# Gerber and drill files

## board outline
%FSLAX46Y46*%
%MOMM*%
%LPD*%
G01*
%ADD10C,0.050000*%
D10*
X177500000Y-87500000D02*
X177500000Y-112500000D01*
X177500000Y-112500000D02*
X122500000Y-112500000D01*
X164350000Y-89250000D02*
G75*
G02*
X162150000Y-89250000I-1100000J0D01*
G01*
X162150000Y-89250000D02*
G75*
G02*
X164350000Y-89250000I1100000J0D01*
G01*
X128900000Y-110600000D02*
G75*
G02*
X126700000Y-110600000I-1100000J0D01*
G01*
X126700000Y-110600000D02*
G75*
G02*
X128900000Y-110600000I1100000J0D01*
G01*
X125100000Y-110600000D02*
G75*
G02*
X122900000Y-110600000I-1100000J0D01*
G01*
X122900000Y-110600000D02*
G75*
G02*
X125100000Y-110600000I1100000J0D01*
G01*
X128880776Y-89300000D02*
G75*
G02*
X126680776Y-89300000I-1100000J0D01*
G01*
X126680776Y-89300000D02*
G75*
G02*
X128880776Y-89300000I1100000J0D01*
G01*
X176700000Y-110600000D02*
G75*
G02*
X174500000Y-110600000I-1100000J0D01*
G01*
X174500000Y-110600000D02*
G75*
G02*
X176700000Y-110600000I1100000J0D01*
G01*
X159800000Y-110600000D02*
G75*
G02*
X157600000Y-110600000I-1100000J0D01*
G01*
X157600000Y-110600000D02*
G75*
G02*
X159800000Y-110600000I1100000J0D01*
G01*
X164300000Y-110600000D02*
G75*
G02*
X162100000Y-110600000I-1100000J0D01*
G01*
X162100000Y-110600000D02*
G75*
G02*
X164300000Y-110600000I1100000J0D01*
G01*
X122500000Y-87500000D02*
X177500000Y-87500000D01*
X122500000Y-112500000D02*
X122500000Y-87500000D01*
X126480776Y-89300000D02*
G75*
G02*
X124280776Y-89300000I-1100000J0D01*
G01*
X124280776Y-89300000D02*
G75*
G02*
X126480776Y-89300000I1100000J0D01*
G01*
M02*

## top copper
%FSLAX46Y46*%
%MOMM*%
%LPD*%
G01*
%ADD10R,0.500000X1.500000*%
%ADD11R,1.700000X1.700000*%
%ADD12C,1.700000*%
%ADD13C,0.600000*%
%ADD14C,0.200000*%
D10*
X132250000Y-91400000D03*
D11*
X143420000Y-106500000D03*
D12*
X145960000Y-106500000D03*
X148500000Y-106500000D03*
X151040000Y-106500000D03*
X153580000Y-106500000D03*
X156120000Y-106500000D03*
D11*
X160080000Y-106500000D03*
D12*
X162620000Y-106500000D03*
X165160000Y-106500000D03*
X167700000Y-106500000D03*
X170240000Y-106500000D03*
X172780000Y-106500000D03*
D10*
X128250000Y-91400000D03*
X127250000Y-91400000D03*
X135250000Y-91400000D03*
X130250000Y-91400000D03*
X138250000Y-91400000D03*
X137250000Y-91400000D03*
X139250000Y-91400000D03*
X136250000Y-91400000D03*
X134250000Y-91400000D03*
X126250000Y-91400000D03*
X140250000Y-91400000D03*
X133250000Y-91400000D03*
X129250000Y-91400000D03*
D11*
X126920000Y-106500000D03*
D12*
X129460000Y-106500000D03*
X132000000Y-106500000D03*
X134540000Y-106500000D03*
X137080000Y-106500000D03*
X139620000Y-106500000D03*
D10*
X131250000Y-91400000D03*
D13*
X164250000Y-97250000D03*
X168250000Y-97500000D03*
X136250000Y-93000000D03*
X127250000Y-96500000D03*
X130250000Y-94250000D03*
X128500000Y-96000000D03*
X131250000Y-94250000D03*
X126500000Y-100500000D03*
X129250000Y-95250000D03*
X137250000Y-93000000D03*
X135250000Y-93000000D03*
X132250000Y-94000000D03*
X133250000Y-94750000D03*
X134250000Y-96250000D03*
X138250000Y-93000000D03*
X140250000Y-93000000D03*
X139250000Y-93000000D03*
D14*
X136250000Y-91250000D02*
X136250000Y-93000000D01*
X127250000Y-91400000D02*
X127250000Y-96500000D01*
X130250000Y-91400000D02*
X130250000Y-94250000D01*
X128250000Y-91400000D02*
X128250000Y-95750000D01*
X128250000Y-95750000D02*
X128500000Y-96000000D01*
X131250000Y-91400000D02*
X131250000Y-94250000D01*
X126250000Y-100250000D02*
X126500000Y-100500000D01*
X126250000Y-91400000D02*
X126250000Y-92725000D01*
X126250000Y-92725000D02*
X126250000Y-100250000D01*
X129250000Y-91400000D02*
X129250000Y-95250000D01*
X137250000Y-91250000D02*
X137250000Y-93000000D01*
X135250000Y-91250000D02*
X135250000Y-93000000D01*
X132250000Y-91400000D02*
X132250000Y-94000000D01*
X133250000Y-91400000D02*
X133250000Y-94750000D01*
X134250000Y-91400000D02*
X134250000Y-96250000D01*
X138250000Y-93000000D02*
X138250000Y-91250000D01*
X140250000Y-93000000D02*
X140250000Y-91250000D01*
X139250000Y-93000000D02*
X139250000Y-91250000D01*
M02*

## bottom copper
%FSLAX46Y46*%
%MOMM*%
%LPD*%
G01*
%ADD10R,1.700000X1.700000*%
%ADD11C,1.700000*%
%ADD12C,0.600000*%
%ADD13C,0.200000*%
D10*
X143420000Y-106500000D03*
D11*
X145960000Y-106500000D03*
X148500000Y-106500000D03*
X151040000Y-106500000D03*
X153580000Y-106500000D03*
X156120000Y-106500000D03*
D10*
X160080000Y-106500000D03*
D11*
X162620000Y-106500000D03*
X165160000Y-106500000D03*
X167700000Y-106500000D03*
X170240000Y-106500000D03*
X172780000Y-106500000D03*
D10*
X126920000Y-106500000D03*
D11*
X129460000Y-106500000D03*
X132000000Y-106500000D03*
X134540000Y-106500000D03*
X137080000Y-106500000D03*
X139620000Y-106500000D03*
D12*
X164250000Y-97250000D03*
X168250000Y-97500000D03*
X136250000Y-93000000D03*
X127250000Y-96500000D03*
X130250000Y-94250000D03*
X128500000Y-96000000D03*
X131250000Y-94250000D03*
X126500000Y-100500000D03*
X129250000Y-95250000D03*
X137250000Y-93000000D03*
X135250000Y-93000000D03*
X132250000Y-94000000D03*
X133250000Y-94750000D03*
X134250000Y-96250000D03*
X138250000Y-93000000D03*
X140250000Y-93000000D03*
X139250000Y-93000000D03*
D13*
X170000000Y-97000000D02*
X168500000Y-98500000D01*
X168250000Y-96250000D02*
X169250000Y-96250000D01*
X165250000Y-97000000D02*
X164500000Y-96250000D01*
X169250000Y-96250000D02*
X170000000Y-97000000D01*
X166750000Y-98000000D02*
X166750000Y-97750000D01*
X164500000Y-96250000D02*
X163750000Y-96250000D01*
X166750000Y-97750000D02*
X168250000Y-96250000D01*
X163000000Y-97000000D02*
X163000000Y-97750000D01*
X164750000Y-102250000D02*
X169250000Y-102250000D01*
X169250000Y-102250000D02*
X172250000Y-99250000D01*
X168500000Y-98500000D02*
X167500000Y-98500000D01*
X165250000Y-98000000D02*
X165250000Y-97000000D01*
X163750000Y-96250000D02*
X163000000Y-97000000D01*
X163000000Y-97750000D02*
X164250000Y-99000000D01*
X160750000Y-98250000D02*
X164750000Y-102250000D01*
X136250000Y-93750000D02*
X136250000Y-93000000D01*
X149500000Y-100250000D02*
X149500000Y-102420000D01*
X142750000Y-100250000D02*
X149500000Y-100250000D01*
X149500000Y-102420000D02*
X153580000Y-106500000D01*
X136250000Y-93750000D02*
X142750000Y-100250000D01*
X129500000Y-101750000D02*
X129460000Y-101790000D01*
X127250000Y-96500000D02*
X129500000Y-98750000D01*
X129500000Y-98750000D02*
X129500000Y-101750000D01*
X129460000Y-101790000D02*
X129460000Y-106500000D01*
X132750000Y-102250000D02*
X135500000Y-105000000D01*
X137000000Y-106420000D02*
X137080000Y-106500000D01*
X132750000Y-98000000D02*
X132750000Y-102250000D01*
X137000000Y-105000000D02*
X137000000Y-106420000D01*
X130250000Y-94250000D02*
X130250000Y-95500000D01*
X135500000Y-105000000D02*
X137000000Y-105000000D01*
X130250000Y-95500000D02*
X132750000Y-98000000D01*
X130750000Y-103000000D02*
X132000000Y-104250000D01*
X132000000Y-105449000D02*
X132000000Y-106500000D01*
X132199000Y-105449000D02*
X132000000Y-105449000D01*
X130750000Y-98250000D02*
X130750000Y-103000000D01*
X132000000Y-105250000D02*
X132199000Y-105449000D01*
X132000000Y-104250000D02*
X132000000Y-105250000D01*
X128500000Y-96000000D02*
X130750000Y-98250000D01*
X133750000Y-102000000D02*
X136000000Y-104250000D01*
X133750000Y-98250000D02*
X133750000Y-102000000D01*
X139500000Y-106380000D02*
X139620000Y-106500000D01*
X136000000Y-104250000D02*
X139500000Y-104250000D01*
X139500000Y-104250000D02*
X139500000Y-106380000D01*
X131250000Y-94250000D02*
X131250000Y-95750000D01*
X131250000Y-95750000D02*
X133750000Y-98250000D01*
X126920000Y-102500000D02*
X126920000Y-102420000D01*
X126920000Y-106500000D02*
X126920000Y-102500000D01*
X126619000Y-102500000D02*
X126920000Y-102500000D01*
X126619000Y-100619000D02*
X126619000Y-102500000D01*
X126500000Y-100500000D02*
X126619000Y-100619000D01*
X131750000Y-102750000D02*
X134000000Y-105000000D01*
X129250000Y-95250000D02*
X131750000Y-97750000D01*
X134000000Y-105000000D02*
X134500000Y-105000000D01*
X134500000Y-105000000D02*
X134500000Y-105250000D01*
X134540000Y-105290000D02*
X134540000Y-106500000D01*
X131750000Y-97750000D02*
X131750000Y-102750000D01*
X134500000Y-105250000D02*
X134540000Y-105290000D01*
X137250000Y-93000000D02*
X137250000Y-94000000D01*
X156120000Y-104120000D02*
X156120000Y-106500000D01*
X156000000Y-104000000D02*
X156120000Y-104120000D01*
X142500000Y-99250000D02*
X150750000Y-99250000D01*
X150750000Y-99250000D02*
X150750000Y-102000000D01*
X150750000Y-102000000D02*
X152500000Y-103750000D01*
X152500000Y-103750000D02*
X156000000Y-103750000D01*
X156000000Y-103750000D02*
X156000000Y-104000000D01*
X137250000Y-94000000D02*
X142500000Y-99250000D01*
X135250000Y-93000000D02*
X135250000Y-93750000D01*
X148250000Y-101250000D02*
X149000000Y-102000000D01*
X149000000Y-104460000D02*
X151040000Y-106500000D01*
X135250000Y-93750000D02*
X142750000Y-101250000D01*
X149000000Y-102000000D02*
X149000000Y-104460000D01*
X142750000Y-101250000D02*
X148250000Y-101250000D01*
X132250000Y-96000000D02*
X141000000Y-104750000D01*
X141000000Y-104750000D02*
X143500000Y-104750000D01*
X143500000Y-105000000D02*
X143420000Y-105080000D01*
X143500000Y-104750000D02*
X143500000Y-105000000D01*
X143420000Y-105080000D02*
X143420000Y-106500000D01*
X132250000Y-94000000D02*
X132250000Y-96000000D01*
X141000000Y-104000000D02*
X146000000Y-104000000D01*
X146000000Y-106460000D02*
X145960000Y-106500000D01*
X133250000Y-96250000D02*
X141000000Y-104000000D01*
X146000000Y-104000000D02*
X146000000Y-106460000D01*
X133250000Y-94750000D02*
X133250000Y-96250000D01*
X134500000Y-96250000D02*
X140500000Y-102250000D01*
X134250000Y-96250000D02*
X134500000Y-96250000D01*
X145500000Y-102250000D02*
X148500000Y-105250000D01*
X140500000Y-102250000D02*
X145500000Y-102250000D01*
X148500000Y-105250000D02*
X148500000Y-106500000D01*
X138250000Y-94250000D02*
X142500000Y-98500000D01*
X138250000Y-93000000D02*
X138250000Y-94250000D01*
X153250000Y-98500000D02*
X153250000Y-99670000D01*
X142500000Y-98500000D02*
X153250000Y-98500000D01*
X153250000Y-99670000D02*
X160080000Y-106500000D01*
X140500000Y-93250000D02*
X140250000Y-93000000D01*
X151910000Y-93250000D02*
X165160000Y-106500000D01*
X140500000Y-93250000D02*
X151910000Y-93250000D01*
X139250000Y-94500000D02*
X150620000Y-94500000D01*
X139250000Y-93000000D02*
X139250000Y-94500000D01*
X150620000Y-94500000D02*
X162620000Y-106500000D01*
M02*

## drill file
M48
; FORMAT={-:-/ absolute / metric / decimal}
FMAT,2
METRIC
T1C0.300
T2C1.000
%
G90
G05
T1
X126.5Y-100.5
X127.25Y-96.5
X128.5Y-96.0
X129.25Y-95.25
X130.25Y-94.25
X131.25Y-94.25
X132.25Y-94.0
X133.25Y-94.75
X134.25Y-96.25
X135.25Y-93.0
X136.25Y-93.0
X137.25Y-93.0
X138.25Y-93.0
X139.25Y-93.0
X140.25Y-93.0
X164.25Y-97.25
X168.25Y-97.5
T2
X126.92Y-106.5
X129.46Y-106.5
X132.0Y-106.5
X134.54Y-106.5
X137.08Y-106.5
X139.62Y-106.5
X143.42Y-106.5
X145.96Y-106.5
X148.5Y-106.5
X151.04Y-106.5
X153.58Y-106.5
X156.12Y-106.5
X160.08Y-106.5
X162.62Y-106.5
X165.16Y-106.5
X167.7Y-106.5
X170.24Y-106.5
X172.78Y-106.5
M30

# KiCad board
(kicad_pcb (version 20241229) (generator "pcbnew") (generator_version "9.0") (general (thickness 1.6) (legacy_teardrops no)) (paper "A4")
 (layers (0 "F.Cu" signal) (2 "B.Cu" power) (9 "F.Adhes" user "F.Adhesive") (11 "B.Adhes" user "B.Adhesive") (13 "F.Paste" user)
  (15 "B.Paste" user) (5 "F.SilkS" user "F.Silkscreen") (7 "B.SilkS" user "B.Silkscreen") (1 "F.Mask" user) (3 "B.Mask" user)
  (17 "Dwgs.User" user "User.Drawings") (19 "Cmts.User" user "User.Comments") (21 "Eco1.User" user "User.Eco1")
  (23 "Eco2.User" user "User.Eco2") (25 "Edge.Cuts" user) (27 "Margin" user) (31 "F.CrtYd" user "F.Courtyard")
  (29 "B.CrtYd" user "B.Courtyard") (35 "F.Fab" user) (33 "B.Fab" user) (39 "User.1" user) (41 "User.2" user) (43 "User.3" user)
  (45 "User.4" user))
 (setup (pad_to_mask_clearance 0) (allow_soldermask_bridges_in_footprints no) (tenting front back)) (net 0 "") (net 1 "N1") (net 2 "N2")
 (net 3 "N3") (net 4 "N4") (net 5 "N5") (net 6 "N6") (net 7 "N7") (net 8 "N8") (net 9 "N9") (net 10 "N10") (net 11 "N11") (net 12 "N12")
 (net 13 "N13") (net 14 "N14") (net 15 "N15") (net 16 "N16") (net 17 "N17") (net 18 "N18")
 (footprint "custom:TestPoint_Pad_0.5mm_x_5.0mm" (layer "F.Cu") (at 132.25 92.15)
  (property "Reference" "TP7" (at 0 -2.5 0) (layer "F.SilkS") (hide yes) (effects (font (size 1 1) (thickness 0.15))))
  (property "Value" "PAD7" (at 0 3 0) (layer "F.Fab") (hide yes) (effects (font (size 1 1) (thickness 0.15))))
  (pad "1" smd rect (at 0 -0.75) (size 0.5 1.5) (layers "F.Cu" "F.Mask" "F.Paste") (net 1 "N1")))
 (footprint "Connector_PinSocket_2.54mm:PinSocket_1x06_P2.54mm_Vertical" (layer "F.Cu") (at 143.42 106.5 90)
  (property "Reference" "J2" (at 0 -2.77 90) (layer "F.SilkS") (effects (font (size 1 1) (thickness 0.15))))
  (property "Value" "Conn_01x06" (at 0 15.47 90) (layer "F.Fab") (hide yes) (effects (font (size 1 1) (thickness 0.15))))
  (pad "1" thru_hole rect (at 0 0 90) (size 1.7 1.7) (drill 1) (layers "*.Cu" "*.Mask") (remove_unused_layers no) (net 1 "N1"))
  (pad "2" thru_hole circle (at 0 2.54 90) (size 1.7 1.7) (drill 1) (layers "*.Cu" "*.Mask") (remove_unused_layers no) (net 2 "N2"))
  (pad "3" thru_hole circle (at 0 5.08 90) (size 1.7 1.7) (drill 1) (layers "*.Cu" "*.Mask") (remove_unused_layers no) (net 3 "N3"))
  (pad "4" thru_hole circle (at 0 7.62 90) (size 1.7 1.7) (drill 1) (layers "*.Cu" "*.Mask") (remove_unused_layers no) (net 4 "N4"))
  (pad "5" thru_hole circle (at 0 10.16 90) (size 1.7 1.7) (drill 1) (layers "*.Cu" "*.Mask") (remove_unused_layers no) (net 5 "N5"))
  (pad "6" thru_hole circle (at 0 12.7 90) (size 1.7 1.7) (drill 1) (layers "*.Cu" "*.Mask") (remove_unused_layers no) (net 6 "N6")))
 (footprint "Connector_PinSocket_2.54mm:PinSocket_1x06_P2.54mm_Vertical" (layer "F.Cu") (at 160.08 106.5 90)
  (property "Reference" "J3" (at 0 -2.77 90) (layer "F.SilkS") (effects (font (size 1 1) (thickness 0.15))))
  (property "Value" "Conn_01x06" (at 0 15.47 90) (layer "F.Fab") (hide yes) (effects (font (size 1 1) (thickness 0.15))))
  (pad "1" thru_hole rect (at 0 0 90) (size 1.7 1.7) (drill 1) (layers "*.Cu" "*.Mask") (remove_unused_layers no) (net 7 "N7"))
  (pad "2" thru_hole circle (at 0 2.54 90) (size 1.7 1.7) (drill 1) (layers "*.Cu" "*.Mask") (remove_unused_layers no) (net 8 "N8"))
  (pad "3" thru_hole circle (at 0 5.08 90) (size 1.7 1.7) (drill 1) (layers "*.Cu" "*.Mask") (remove_unused_layers no) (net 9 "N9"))
  (pad "4" thru_hole circle (at 0 7.62 90) (size 1.7 1.7) (drill 1) (layers "*.Cu" "*.Mask") (remove_unused_layers no) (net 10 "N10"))
  (pad "5" thru_hole circle (at 0 10.16 90) (size 1.7 1.7) (drill 1) (layers "*.Cu" "*.Mask") (remove_unused_layers no) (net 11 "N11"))
  (pad "6" thru_hole circle (at 0 12.7 90) (size 1.7 1.7) (drill 1) (layers "*.Cu" "*.Mask") (remove_unused_layers no) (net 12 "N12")))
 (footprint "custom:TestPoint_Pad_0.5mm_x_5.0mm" (layer "F.Cu") (at 128.25 92.15)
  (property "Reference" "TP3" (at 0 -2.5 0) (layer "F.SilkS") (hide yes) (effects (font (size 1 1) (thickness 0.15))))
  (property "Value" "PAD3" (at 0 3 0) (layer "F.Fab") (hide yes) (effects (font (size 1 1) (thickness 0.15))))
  (pad "1" smd rect (at 0 -0.75) (size 0.5 1.5) (layers "F.Cu" "F.Mask" "F.Paste") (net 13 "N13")))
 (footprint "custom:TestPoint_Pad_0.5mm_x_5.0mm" (layer "F.Cu") (at 127.25 92.15)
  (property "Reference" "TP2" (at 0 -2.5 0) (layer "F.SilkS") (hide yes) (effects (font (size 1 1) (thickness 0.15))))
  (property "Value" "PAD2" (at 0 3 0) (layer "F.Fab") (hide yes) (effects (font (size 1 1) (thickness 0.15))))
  (pad "1" smd rect (at 0 -0.75) (size 0.5 1.5) (layers "F.Cu" "F.Mask" "F.Paste") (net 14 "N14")))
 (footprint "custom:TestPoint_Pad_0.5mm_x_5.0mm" (layer "F.Cu") (at 135.25 92.15)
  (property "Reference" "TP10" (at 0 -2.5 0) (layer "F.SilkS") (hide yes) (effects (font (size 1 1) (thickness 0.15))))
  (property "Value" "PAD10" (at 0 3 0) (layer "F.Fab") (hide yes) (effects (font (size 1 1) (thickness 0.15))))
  (pad "1" smd rect (at 0 -0.75) (size 0.5 1.5) (layers "F.Cu" "F.Mask" "F.Paste") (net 4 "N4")))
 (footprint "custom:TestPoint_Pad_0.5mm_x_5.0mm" (layer "F.Cu") (at 130.25 92.15)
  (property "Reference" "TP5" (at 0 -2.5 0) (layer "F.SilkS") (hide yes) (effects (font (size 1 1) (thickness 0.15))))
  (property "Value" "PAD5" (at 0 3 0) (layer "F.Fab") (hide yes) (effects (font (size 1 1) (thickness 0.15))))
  (pad "1" smd rect (at 0 -0.75) (size 0.5 1.5) (layers "F.Cu" "F.Mask" "F.Paste") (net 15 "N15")))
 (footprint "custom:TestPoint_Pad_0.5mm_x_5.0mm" (layer "F.Cu") (at 138.25 92.15)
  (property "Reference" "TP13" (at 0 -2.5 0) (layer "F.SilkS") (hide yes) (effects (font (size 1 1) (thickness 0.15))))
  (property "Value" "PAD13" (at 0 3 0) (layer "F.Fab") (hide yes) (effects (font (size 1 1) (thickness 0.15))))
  (pad "1" smd rect (at 0 -0.75) (size 0.5 1.5) (layers "F.Cu" "F.Mask" "F.Paste") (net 7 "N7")))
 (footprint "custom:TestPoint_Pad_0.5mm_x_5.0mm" (layer "F.Cu") (at 137.25 92.15)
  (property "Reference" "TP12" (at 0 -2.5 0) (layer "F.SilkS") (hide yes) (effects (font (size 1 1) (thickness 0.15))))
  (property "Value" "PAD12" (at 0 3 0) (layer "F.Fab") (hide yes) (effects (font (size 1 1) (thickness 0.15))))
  (pad "1" smd rect (at 0 -0.75) (size 0.5 1.5) (layers "F.Cu" "F.Mask" "F.Paste") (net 6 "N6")))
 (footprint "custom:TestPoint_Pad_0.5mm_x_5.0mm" (layer "F.Cu") (at 139.25 92.15)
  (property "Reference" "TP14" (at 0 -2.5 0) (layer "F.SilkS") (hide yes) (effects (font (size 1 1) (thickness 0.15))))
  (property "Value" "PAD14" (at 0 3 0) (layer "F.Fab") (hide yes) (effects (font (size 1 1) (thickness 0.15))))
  (pad "1" smd rect (at 0 -0.75) (size 0.5 1.5) (layers "F.Cu" "F.Mask" "F.Paste") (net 8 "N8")))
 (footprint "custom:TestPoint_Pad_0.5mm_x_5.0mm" (layer "F.Cu") (at 136.25 92.15)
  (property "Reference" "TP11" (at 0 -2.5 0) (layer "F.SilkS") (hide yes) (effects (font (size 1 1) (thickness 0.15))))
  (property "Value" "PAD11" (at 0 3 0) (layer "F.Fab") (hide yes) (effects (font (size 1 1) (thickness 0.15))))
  (pad "1" smd rect (at 0 -0.75) (size 0.5 1.5) (layers "F.Cu" "F.Mask" "F.Paste") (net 5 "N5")))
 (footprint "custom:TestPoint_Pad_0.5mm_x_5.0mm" (layer "F.Cu") (at 134.25 92.15)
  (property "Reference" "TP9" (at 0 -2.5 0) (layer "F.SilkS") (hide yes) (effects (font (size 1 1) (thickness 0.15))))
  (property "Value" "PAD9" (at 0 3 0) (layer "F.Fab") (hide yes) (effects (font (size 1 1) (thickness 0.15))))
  (pad "1" smd rect (at 0 -0.75) (size 0.5 1.5) (layers "F.Cu" "F.Mask" "F.Paste") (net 3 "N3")))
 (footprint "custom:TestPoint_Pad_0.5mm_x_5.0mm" (layer "F.Cu") (at 126.25 92.15)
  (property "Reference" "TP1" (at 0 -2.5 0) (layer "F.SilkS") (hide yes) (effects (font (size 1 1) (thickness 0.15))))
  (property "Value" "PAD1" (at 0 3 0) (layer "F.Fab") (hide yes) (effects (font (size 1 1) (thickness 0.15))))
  (pad "1" smd rect (at 0 -0.75) (size 0.5 1.5) (layers "F.Cu" "F.Mask" "F.Paste") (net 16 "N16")))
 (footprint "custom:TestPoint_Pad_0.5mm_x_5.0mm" (layer "F.Cu") (at 140.25 92.15)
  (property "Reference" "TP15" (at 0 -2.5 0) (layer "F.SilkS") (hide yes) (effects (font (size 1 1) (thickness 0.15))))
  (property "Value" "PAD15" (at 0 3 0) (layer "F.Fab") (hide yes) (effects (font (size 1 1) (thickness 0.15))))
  (pad "1" smd rect (at 0 -0.75) (size 0.5 1.5) (layers "F.Cu" "F.Mask" "F.Paste") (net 9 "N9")))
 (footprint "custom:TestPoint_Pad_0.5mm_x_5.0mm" (layer "F.Cu") (at 133.25 92.15)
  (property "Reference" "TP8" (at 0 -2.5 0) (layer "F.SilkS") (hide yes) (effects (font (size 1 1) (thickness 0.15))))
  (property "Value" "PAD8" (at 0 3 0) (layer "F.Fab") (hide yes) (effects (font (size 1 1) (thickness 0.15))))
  (pad "1" smd rect (at 0 -0.75) (size 0.5 1.5) (layers "F.Cu" "F.Mask" "F.Paste") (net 2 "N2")))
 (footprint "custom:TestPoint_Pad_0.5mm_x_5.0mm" (layer "F.Cu") (at 129.25 92.15)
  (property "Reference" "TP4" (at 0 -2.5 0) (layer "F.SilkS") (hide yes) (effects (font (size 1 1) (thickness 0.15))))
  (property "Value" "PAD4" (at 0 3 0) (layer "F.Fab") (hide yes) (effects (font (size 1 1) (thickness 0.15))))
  (pad "1" smd rect (at 0 -0.75) (size 0.5 1.5) (layers "F.Cu" "F.Mask" "F.Paste") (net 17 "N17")))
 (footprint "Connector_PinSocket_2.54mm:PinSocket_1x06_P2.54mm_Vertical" (layer "F.Cu") (at 126.92 106.5 90)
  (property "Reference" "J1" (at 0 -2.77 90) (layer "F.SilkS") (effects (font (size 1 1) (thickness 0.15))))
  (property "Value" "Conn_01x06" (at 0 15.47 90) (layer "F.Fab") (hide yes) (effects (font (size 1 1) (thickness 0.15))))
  (pad "1" thru_hole rect (at 0 0 90) (size 1.7 1.7) (drill 1) (layers "*.Cu" "*.Mask") (remove_unused_layers no) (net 16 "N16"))
  (pad "2" thru_hole circle (at 0 2.54 90) (size 1.7 1.7) (drill 1) (layers "*.Cu" "*.Mask") (remove_unused_layers no) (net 14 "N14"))
  (pad "3" thru_hole circle (at 0 5.08 90) (size 1.7 1.7) (drill 1) (layers "*.Cu" "*.Mask") (remove_unused_layers no) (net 13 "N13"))
  (pad "4" thru_hole circle (at 0 7.62 90) (size 1.7 1.7) (drill 1) (layers "*.Cu" "*.Mask") (remove_unused_layers no) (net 17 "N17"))
  (pad "5" thru_hole circle (at 0 10.16 90) (size 1.7 1.7) (drill 1) (layers "*.Cu" "*.Mask") (remove_unused_layers no) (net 15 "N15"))
  (pad "6" thru_hole circle (at 0 12.7 90) (size 1.7 1.7) (drill 1) (layers "*.Cu" "*.Mask") (remove_unused_layers no) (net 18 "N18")))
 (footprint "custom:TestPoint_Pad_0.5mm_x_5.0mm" (layer "F.Cu") (at 131.25 92.15)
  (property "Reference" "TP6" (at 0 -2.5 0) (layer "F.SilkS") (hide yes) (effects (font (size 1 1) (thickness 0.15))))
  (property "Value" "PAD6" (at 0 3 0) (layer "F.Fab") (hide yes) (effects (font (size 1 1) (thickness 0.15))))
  (pad "1" smd rect (at 0 -0.75) (size 0.5 1.5) (layers "F.Cu" "F.Mask" "F.Paste") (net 18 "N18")))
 (gr_line (start 177.5 87.5) (end 177.5 112.5) (stroke (width 0.05) (type default)) (layer "Edge.Cuts"))
 (gr_line (start 177.5 112.5) (end 122.5 112.5) (stroke (width 0.05) (type default)) (layer "Edge.Cuts"))
 (gr_circle (center 163.25 89.25) (end 164.35 89.25) (stroke (width 0.05) (type solid)) (fill no) (layer "Edge.Cuts"))
 (gr_circle (center 127.8 110.6) (end 128.9 110.6) (stroke (width 0.05) (type solid)) (fill no) (layer "Edge.Cuts"))
 (gr_circle (center 124 110.6) (end 125.1 110.6) (stroke (width 0.05) (type solid)) (fill no) (layer "Edge.Cuts"))
 (gr_circle (center 127.780776 89.3) (end 128.880776 89.3) (stroke (width 0.05) (type solid)) (fill no) (layer "Edge.Cuts"))
 (gr_circle (center 175.6 110.6) (end 176.7 110.6) (stroke (width 0.05) (type solid)) (fill no) (layer "Edge.Cuts"))
 (gr_circle (center 158.7 110.6) (end 159.8 110.6) (stroke (width 0.05) (type solid)) (fill no) (layer "Edge.Cuts"))
 (gr_circle (center 163.2 110.6) (end 164.3 110.6) (stroke (width 0.05) (type solid)) (fill no) (layer "Edge.Cuts"))
 (gr_line (start 122.5 87.5) (end 177.5 87.5) (stroke (width 0.05) (type solid)) (layer "Edge.Cuts"))
 (gr_line (start 122.5 112.5) (end 122.5 87.5) (stroke (width 0.05) (type default)) (layer "Edge.Cuts"))
 (gr_circle (center 125.380776 89.3) (end 126.480776 89.3) (stroke (width 0.05) (type solid)) (fill no) (layer "Edge.Cuts"))
 (via (at 164.25 97.25) (size 0.6) (drill 0.3) (layers "F.Cu" "B.Cu") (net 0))
 (via (at 168.25 97.5) (size 0.6) (drill 0.3) (layers "F.Cu" "B.Cu") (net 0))
 (segment (start 170 97) (end 168.5 98.5) (width 0.2) (layer "B.Cu") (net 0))
 (segment (start 168.25 96.25) (end 169.25 96.25) (width 0.2) (layer "B.Cu") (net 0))
 (segment (start 165.25 97) (end 164.5 96.25) (width 0.2) (layer "B.Cu") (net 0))
 (segment (start 169.25 96.25) (end 170 97) (width 0.2) (layer "B.Cu") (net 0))
 (segment (start 166.75 98) (end 166.75 97.75) (width 0.2) (layer "B.Cu") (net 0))
 (segment (start 164.5 96.25) (end 163.75 96.25) (width 0.2) (layer "B.Cu") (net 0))
 (segment (start 166.75 97.75) (end 168.25 96.25) (width 0.2) (layer "B.Cu") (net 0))
 (segment (start 163 97) (end 163 97.75) (width 0.2) (layer "B.Cu") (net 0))
 (segment (start 164.75 102.25) (end 169.25 102.25) (width 0.2) (layer "B.Cu") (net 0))
 (segment (start 169.25 102.25) (end 172.25 99.25) (width 0.2) (layer "B.Cu") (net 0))
 (segment (start 168.5 98.5) (end 167.5 98.5) (width 0.2) (layer "B.Cu") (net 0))
 (segment (start 165.25 98) (end 165.25 97) (width 0.2) (layer "B.Cu") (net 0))
 (segment (start 163.75 96.25) (end 163 97) (width 0.2) (layer "B.Cu") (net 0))
 (segment (start 163 97.75) (end 164.25 99) (width 0.2) (layer "B.Cu") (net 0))
 (segment (start 160.75 98.25) (end 164.75 102.25) (width 0.2) (layer "B.Cu") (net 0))
 (segment (start 136.25 91.25) (end 136.25 93) (width 0.2) (layer "F.Cu") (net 5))
 (via (at 136.25 93) (size 0.6) (drill 0.3) (layers "F.Cu" "B.Cu") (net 5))
 (segment (start 136.25 93.75) (end 136.25 93) (width 0.2) (layer "B.Cu") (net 5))
 (segment (start 149.5 100.25) (end 149.5 102.42) (width 0.2) (layer "B.Cu") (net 5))
 (segment (start 142.75 100.25) (end 149.5 100.25) (width 0.2) (layer "B.Cu") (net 5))
 (segment (start 149.5 102.42) (end 153.58 106.5) (width 0.2) (layer "B.Cu") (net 5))
 (segment (start 136.25 93.75) (end 142.75 100.25) (width 0.2) (layer "B.Cu") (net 5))
 (segment (start 127.25 91.4) (end 127.25 96.5) (width 0.2) (layer "F.Cu") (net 14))
 (via (at 127.25 96.5) (size 0.6) (drill 0.3) (layers "F.Cu" "B.Cu") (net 14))
 (segment (start 129.5 101.75) (end 129.46 101.79) (width 0.2) (layer "B.Cu") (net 14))
 (segment (start 127.25 96.5) (end 129.5 98.75) (width 0.2) (layer "B.Cu") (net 14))
 (segment (start 129.5 98.75) (end 129.5 101.75) (width 0.2) (layer "B.Cu") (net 14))
 (segment (start 129.46 101.79) (end 129.46 106.5) (width 0.2) (layer "B.Cu") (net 14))
 (segment (start 130.25 91.4) (end 130.25 94.25) (width 0.2) (layer "F.Cu") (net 15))
 (via (at 130.25 94.25) (size 0.6) (drill 0.3) (layers "F.Cu" "B.Cu") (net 15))
 (segment (start 132.75 102.25) (end 135.5 105) (width 0.2) (layer "B.Cu") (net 15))
 (segment (start 137 106.42) (end 137.08 106.5) (width 0.2) (layer "B.Cu") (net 15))
 (segment (start 132.75 98) (end 132.75 102.25) (width 0.2) (layer "B.Cu") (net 15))
 (segment (start 137 105) (end 137 106.42) (width 0.2) (layer "B.Cu") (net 15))
 (segment (start 130.25 94.25) (end 130.25 95.5) (width 0.2) (layer "B.Cu") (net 15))
 (segment (start 135.5 105) (end 137 105) (width 0.2) (layer "B.Cu") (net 15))
 (segment (start 130.25 95.5) (end 132.75 98) (width 0.2) (layer "B.Cu") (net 15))
 (segment (start 128.25 91.4) (end 128.25 95.75) (width 0.2) (layer "F.Cu") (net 13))
 (segment (start 128.25 95.75) (end 128.5 96) (width 0.2) (layer "F.Cu") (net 13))
 (via (at 128.5 96) (size 0.6) (drill 0.3) (layers "F.Cu" "B.Cu") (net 13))
 (segment (start 130.75 103) (end 132 104.25) (width 0.2) (layer "B.Cu") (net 13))
 (segment (start 132 105.449) (end 132 106.5) (width 0.2) (layer "B.Cu") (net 13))
 (segment (start 132.199 105.449) (end 132 105.449) (width 0.2) (layer "B.Cu") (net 13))
 (segment (start 130.75 98.25) (end 130.75 103) (width 0.2) (layer "B.Cu") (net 13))
 (segment (start 132 105.25) (end 132.199 105.449) (width 0.2) (layer "B.Cu") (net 13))
 (segment (start 132 104.25) (end 132 105.25) (width 0.2) (layer "B.Cu") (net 13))
 (segment (start 128.5 96) (end 130.75 98.25) (width 0.2) (layer "B.Cu") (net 13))
 (segment (start 131.25 91.4) (end 131.25 94.25) (width 0.2) (layer "F.Cu") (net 18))
 (via (at 131.25 94.25) (size 0.6) (drill 0.3) (layers "F.Cu" "B.Cu") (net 18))
 (segment (start 133.75 102) (end 136 104.25) (width 0.2) (layer "B.Cu") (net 18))
 (segment (start 133.75 98.25) (end 133.75 102) (width 0.2) (layer "B.Cu") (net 18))
 (segment (start 139.5 106.38) (end 139.62 106.5) (width 0.2) (layer "B.Cu") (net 18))
 (segment (start 136 104.25) (end 139.5 104.25) (width 0.2) (layer "B.Cu") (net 18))
 (segment (start 139.5 104.25) (end 139.5 106.38) (width 0.2) (layer "B.Cu") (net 18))
 (segment (start 131.25 94.25) (end 131.25 95.75) (width 0.2) (layer "B.Cu") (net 18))
 (segment (start 131.25 95.75) (end 133.75 98.25) (width 0.2) (layer "B.Cu") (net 18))
 (segment (start 126.25 100.25) (end 126.5 100.5) (width 0.2) (layer "F.Cu") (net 16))
 (segment (start 126.25 91.4) (end 126.25 92.725) (width 0.2) (layer "F.Cu") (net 16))
 (segment (start 126.25 92.725) (end 126.25 100.25) (width 0.2) (layer "F.Cu") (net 16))
 (via (at 126.5 100.5) (size 0.6) (drill 0.3) (layers "F.Cu" "B.Cu") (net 16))
 (segment (start 126.92 102.5) (end 126.92 102.42) (width 0.2) (layer "B.Cu") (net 16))
 (segment (start 126.92 106.5) (end 126.92 102.5) (width 0.2) (layer "B.Cu") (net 16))
 (segment (start 126.619 102.5) (end 126.92 102.5) (width 0.2) (layer "B.Cu") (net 16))
 (segment (start 126.619 100.619) (end 126.619 102.5) (width 0.2) (layer "B.Cu") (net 16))
 (segment (start 126.5 100.5) (end 126.619 100.619) (width 0.2) (layer "B.Cu") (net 16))
 (segment (start 129.25 91.4) (end 129.25 95.25) (width 0.2) (layer "F.Cu") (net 17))
 (via (at 129.25 95.25) (size 0.6) (drill 0.3) (layers "F.Cu" "B.Cu") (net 17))
 (segment (start 131.75 102.75) (end 134 105) (width 0.2) (layer "B.Cu") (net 17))
 (segment (start 129.25 95.25) (end 131.75 97.75) (width 0.2) (layer "B.Cu") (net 17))
 (segment (start 134 105) (end 134.5 105) (width 0.2) (layer "B.Cu") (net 17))
 (segment (start 134.5 105) (end 134.5 105.25) (width 0.2) (layer "B.Cu") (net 17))
 (segment (start 134.54 105.29) (end 134.54 106.5) (width 0.2) (layer "B.Cu") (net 17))
 (segment (start 131.75 97.75) (end 131.75 102.75) (width 0.2) (layer "B.Cu") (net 17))
 (segment (start 134.5 105.25) (end 134.54 105.29) (width 0.2) (layer "B.Cu") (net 17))
 (segment (start 137.25 91.25) (end 137.25 93) (width 0.2) (layer "F.Cu") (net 6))
 (via (at 137.25 93) (size 0.6) (drill 0.3) (layers "F.Cu" "B.Cu") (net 6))
 (segment (start 137.25 93) (end 137.25 94) (width 0.2) (layer "B.Cu") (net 6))
 (segment (start 156.12 104.12) (end 156.12 106.5) (width 0.2) (layer "B.Cu") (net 6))
 (segment (start 156 104) (end 156.12 104.12) (width 0.2) (layer "B.Cu") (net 6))
 (segment (start 142.5 99.25) (end 150.75 99.25) (width 0.2) (layer "B.Cu") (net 6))
 (segment (start 150.75 99.25) (end 150.75 102) (width 0.2) (layer "B.Cu") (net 6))
 (segment (start 150.75 102) (end 152.5 103.75) (width 0.2) (layer "B.Cu") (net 6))
 (segment (start 152.5 103.75) (end 156 103.75) (width 0.2) (layer "B.Cu") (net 6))
 (segment (start 156 103.75) (end 156 104) (width 0.2) (layer "B.Cu") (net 6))
 (segment (start 137.25 94) (end 142.5 99.25) (width 0.2) (layer "B.Cu") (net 6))
 (segment (start 135.25 91.25) (end 135.25 93) (width 0.2) (layer "F.Cu") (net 4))
 (via (at 135.25 93) (size 0.6) (drill 0.3) (layers "F.Cu" "B.Cu") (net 4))
 (segment (start 135.25 93) (end 135.25 93.75) (width 0.2) (layer "B.Cu") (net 4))
 (segment (start 148.25 101.25) (end 149 102) (width 0.2) (layer "B.Cu") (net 4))
 (segment (start 149 104.46) (end 151.04 106.5) (width 0.2) (layer "B.Cu") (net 4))
 (segment (start 135.25 93.75) (end 142.75 101.25) (width 0.2) (layer "B.Cu") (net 4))
 (segment (start 149 102) (end 149 104.46) (width 0.2) (layer "B.Cu") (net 4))
 (segment (start 142.75 101.25) (end 148.25 101.25) (width 0.2) (layer "B.Cu") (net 4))
 (segment (start 132.25 91.4) (end 132.25 94) (width 0.2) (layer "F.Cu") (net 1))
 (via (at 132.25 94) (size 0.6) (drill 0.3) (layers "F.Cu" "B.Cu") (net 1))
 (segment (start 132.25 96) (end 141 104.75) (width 0.2) (layer "B.Cu") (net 1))
 (segment (start 141 104.75) (end 143.5 104.75) (width 0.2) (layer "B.Cu") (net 1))
 (segment (start 143.5 105) (end 143.42 105.08) (width 0.2) (layer "B.Cu") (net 1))
 (segment (start 143.5 104.75) (end 143.5 105) (width 0.2) (layer "B.Cu") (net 1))
 (segment (start 143.42 105.08) (end 143.42 106.5) (width 0.2) (layer "B.Cu") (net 1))
 (segment (start 132.25 94) (end 132.25 96) (width 0.2) (layer "B.Cu") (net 1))
 (segment (start 133.25 91.4) (end 133.25 94.75) (width 0.2) (layer "F.Cu") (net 2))
 (via (at 133.25 94.75) (size 0.6) (drill 0.3) (layers "F.Cu" "B.Cu") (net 2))
 (segment (start 141 104) (end 146 104) (width 0.2) (layer "B.Cu") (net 2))
 (segment (start 146 106.46) (end 145.96 106.5) (width 0.2) (layer "B.Cu") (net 2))
 (segment (start 133.25 96.25) (end 141 104) (width 0.2) (layer "B.Cu") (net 2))
 (segment (start 146 104) (end 146 106.46) (width 0.2) (layer "B.Cu") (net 2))
 (segment (start 133.25 94.75) (end 133.25 96.25) (width 0.2) (layer "B.Cu") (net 2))
 (segment (start 134.25 91.4) (end 134.25 96.25) (width 0.2) (layer "F.Cu") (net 3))
 (via (at 134.25 96.25) (size 0.6) (drill 0.3) (layers "F.Cu" "B.Cu") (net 3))
 (segment (start 134.5 96.25) (end 140.5 102.25) (width 0.2) (layer "B.Cu") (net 3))
 (segment (start 134.25 96.25) (end 134.5 96.25) (width 0.2) (layer "B.Cu") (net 3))
 (segment (start 145.5 102.25) (end 148.5 105.25) (width 0.2) (layer "B.Cu") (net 3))
 (segment (start 140.5 102.25) (end 145.5 102.25) (width 0.2) (layer "B.Cu") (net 3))
 (segment (start 148.5 105.25) (end 148.5 106.5) (width 0.2) (layer "B.Cu") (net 3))
 (segment (start 138.25 93) (end 138.25 91.25) (width 0.2) (layer "F.Cu") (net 7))
 (via (at 138.25 93) (size 0.6) (drill 0.3) (layers "F.Cu" "B.Cu") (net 7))
 (segment (start 138.25 94.25) (end 142.5 98.5) (width 0.2) (layer "B.Cu") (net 7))
 (segment (start 138.25 93) (end 138.25 94.25) (width 0.2) (layer "B.Cu") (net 7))
 (segment (start 153.25 98.5) (end 153.25 99.67) (width 0.2) (layer "B.Cu") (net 7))
 (segment (start 142.5 98.5) (end 153.25 98.5) (width 0.2) (layer "B.Cu") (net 7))
 (segment (start 153.25 99.67) (end 160.08 106.5) (width 0.2) (layer "B.Cu") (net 7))
 (segment (start 140.25 93) (end 140.25 91.25) (width 0.2) (layer "F.Cu") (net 9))
 (via (at 140.25 93) (size 0.6) (drill 0.3) (layers "F.Cu" "B.Cu") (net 9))
 (segment (start 140.5 93.25) (end 140.25 93) (width 0.2) (layer "B.Cu") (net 9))
 (segment (start 151.91 93.25) (end 165.16 106.5) (width 0.2) (layer "B.Cu") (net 9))
 (segment (start 140.5 93.25) (end 151.91 93.25) (width 0.2) (layer "B.Cu") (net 9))
 (segment (start 139.25 93) (end 139.25 91.25) (width 0.2) (layer "F.Cu") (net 8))
 (via (at 139.25 93) (size 0.6) (drill 0.3) (layers "F.Cu" "B.Cu") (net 8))
 (segment (start 139.25 94.5) (end 150.62 94.5) (width 0.2) (layer "B.Cu") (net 8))
 (segment (start 139.25 93) (end 139.25 94.5) (width 0.2) (layer "B.Cu") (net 8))
 (segment (start 150.62 94.5) (end 162.62 106.5) (width 0.2) (layer "B.Cu") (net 8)))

